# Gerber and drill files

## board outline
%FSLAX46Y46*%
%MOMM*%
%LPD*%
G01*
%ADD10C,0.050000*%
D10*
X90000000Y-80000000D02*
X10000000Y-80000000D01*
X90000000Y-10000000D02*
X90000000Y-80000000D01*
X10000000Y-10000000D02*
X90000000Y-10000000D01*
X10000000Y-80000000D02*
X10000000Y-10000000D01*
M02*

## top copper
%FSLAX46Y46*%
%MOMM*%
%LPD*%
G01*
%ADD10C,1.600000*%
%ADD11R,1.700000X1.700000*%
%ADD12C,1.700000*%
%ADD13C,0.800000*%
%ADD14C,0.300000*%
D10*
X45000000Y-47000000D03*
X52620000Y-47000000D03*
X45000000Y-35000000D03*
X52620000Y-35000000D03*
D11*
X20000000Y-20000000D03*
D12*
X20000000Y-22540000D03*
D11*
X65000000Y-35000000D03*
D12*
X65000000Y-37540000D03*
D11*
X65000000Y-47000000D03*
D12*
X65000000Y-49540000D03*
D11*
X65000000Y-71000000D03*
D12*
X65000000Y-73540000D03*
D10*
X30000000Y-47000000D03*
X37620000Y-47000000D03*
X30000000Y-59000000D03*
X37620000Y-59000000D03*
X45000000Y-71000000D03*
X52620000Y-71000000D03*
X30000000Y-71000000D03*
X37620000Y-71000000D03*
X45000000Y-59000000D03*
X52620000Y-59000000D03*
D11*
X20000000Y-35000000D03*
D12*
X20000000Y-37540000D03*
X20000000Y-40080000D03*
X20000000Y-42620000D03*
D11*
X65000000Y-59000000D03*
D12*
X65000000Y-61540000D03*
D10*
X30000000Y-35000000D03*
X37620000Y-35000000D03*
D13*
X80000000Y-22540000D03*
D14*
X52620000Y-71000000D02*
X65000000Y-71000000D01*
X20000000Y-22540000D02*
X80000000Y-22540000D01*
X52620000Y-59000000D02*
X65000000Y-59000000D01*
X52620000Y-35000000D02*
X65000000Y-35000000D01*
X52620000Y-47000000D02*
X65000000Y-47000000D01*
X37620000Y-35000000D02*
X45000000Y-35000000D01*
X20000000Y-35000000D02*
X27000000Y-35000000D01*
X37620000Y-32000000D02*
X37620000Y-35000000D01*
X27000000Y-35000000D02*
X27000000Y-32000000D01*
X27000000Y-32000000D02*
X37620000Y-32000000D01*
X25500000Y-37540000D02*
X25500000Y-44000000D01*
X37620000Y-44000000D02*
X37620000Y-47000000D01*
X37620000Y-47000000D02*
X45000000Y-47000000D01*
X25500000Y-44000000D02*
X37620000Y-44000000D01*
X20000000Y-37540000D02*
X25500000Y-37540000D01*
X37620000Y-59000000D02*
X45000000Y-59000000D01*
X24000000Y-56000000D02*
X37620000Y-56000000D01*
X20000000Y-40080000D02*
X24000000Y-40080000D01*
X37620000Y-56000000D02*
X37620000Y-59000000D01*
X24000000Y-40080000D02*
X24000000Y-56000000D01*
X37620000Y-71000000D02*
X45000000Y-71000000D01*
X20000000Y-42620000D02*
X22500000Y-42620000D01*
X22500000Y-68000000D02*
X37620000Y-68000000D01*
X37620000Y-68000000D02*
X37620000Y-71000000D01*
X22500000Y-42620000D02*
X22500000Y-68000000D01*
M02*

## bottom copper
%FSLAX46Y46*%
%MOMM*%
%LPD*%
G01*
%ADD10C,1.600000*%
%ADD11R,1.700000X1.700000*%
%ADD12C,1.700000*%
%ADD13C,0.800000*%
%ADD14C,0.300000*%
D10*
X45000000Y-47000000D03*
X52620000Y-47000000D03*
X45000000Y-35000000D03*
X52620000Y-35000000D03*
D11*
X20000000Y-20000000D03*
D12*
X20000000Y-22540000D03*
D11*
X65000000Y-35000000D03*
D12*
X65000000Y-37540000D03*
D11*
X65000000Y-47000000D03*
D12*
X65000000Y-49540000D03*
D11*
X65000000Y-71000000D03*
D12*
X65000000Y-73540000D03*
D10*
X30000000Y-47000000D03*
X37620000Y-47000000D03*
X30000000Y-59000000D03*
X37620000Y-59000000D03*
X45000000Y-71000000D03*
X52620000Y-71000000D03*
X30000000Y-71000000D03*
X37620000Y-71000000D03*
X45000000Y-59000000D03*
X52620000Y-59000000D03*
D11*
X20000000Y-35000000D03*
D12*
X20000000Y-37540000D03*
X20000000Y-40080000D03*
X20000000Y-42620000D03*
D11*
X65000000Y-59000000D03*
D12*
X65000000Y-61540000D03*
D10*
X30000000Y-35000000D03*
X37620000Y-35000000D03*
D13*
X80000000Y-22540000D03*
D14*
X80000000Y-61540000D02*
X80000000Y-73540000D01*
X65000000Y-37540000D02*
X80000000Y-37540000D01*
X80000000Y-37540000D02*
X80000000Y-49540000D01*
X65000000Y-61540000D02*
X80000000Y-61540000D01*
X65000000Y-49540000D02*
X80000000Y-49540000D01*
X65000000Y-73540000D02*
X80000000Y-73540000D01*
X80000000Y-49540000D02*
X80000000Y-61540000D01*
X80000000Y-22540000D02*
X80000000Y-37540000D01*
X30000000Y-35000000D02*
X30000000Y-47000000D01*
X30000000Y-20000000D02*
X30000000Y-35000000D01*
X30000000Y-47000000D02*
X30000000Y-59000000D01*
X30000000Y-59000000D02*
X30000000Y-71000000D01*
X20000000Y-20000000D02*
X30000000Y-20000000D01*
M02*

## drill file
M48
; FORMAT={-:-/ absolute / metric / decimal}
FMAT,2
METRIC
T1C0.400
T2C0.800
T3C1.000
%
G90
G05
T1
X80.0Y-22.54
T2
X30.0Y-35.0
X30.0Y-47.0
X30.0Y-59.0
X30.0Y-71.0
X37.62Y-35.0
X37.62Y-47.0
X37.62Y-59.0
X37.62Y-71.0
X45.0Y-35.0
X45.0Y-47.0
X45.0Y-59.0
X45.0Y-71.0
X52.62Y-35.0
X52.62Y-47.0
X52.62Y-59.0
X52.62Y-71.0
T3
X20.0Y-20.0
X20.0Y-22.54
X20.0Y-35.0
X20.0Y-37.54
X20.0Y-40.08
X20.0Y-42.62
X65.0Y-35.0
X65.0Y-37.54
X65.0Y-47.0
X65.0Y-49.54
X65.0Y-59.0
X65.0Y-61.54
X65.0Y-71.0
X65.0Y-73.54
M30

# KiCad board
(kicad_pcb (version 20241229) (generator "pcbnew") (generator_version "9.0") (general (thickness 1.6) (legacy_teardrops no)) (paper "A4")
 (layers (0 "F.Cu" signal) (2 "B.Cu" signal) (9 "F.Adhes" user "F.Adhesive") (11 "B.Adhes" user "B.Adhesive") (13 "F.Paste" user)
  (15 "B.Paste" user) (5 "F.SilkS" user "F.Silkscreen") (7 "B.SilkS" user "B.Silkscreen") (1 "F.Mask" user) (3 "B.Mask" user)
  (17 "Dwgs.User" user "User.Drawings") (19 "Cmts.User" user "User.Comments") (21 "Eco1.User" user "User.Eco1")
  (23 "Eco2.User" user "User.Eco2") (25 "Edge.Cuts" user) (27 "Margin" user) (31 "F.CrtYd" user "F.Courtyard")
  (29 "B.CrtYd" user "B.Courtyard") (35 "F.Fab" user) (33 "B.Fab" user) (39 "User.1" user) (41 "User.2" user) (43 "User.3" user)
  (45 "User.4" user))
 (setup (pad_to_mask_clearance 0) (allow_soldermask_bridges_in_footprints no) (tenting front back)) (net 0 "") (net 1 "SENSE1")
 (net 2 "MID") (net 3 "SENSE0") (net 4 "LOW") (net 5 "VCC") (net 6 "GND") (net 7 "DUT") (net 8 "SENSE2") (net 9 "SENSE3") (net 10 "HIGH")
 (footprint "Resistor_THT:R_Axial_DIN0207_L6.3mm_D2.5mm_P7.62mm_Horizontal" (layer "F.Cu") (at 45 47)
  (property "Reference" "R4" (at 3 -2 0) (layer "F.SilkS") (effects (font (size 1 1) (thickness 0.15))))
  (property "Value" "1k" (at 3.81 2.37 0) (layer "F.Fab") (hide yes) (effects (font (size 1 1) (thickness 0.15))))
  (pad "1" thru_hole circle (at 0 0) (size 1.6 1.6) (drill 0.8) (layers "*.Cu" "*.Mask") (remove_unused_layers no) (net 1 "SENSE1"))
  (pad "2" thru_hole circle (at 7.62 0) (size 1.6 1.6) (drill 0.8) (layers "*.Cu" "*.Mask") (remove_unused_layers no) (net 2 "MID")))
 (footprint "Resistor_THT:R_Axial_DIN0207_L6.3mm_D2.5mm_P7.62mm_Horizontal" (layer "F.Cu") (at 45 35)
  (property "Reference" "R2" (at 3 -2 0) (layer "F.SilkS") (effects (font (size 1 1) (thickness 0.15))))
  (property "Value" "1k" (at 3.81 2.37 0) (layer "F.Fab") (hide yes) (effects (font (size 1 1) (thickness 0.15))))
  (pad "1" thru_hole circle (at 0 0) (size 1.6 1.6) (drill 0.8) (layers "*.Cu" "*.Mask") (remove_unused_layers no) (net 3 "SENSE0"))
  (pad "2" thru_hole circle (at 7.62 0) (size 1.6 1.6) (drill 0.8) (layers "*.Cu" "*.Mask") (remove_unused_layers no) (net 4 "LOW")))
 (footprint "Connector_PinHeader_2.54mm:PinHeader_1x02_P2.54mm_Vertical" (layer "F.Cu") (at 20 20)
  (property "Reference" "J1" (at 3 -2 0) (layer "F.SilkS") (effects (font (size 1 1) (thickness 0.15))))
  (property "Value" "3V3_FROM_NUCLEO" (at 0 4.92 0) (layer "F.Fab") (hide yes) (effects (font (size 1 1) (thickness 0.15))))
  (pad "1" thru_hole rect (at 0 0) (size 1.7 1.7) (drill 1) (layers "*.Cu" "*.Mask") (remove_unused_layers no) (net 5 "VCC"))
  (pad "2" thru_hole circle (at 0 2.54) (size 1.7 1.7) (drill 1) (layers "*.Cu" "*.Mask") (remove_unused_layers no) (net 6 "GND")))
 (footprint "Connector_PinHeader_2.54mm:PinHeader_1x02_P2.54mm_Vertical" (layer "F.Cu") (at 65 35)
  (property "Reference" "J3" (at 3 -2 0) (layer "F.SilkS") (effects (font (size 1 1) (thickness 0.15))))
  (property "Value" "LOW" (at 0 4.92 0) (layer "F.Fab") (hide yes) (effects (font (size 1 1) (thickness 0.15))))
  (pad "1" thru_hole rect (at 0 0) (size 1.7 1.7) (drill 1) (layers "*.Cu" "*.Mask") (remove_unused_layers no) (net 4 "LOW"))
  (pad "2" thru_hole circle (at 0 2.54) (size 1.7 1.7) (drill 1) (layers "*.Cu" "*.Mask") (remove_unused_layers no) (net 6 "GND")))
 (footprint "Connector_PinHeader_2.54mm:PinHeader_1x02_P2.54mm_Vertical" (layer "F.Cu") (at 65 47)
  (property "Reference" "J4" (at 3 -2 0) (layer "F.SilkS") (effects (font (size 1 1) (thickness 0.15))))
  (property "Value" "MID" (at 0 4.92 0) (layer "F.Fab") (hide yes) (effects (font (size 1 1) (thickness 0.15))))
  (pad "1" thru_hole rect (at 0 0) (size 1.7 1.7) (drill 1) (layers "*.Cu" "*.Mask") (remove_unused_layers no) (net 2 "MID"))
  (pad "2" thru_hole circle (at 0 2.54) (size 1.7 1.7) (drill 1) (layers "*.Cu" "*.Mask") (remove_unused_layers no) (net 6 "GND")))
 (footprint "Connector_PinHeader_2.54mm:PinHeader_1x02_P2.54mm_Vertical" (layer "F.Cu") (at 65 71)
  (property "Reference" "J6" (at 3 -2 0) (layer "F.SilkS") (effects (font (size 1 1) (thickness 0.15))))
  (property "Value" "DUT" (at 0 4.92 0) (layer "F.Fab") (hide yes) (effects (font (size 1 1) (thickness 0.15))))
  (pad "1" thru_hole rect (at 0 0) (size 1.7 1.7) (drill 1) (layers "*.Cu" "*.Mask") (remove_unused_layers no) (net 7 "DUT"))
  (pad "2" thru_hole circle (at 0 2.54) (size 1.7 1.7) (drill 1) (layers "*.Cu" "*.Mask") (remove_unused_layers no) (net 6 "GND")))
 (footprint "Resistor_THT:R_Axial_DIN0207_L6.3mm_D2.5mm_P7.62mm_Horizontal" (layer "F.Cu") (at 30 47)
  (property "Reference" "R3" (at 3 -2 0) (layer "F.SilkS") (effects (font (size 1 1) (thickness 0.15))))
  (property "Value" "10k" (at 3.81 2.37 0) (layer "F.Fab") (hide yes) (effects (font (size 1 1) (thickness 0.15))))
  (pad "1" thru_hole circle (at 0 0) (size 1.6 1.6) (drill 0.8) (layers "*.Cu" "*.Mask") (remove_unused_layers no) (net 5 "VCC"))
  (pad "2" thru_hole circle (at 7.62 0) (size 1.6 1.6) (drill 0.8) (layers "*.Cu" "*.Mask") (remove_unused_layers no) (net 1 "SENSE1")))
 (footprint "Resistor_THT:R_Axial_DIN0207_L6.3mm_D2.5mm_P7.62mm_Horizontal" (layer "F.Cu") (at 30 59)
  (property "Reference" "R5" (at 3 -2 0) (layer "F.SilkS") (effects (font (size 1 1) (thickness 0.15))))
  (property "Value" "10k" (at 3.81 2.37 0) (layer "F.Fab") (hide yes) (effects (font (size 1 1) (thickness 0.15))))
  (pad "1" thru_hole circle (at 0 0) (size 1.6 1.6) (drill 0.8) (layers "*.Cu" "*.Mask") (remove_unused_layers no) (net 5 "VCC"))
  (pad "2" thru_hole circle (at 7.62 0) (size 1.6 1.6) (drill 0.8) (layers "*.Cu" "*.Mask") (remove_unused_layers no) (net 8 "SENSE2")))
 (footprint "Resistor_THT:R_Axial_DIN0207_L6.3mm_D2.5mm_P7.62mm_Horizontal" (layer "F.Cu") (at 45 71)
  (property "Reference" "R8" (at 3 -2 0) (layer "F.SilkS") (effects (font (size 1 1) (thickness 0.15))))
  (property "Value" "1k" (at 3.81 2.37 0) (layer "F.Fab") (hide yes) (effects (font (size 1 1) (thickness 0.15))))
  (pad "1" thru_hole circle (at 0 0) (size 1.6 1.6) (drill 0.8) (layers "*.Cu" "*.Mask") (remove_unused_layers no) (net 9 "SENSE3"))
  (pad "2" thru_hole circle (at 7.62 0) (size 1.6 1.6) (drill 0.8) (layers "*.Cu" "*.Mask") (remove_unused_layers no) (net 7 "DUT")))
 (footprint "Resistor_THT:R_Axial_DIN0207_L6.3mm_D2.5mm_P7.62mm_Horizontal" (layer "F.Cu") (at 30 71)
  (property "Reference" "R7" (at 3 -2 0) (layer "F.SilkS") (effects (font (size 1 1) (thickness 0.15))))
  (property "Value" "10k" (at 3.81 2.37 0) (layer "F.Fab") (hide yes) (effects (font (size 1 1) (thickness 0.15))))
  (pad "1" thru_hole circle (at 0 0) (size 1.6 1.6) (drill 0.8) (layers "*.Cu" "*.Mask") (remove_unused_layers no) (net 5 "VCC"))
  (pad "2" thru_hole circle (at 7.62 0) (size 1.6 1.6) (drill 0.8) (layers "*.Cu" "*.Mask") (remove_unused_layers no) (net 9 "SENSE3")))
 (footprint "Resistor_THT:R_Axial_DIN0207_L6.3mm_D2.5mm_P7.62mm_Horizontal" (layer "F.Cu") (at 45 59)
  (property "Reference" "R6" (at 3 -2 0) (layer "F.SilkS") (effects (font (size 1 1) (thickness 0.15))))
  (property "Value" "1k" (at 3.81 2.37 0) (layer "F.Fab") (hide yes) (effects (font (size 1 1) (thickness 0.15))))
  (pad "1" thru_hole circle (at 0 0) (size 1.6 1.6) (drill 0.8) (layers "*.Cu" "*.Mask") (remove_unused_layers no) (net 8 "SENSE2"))
  (pad "2" thru_hole circle (at 7.62 0) (size 1.6 1.6) (drill 0.8) (layers "*.Cu" "*.Mask") (remove_unused_layers no) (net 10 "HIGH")))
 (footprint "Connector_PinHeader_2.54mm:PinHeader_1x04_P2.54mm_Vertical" (layer "F.Cu") (at 20 35)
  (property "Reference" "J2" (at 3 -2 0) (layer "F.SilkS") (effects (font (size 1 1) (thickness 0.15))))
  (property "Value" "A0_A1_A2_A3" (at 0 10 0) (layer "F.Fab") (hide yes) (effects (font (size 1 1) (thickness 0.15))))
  (pad "1" thru_hole rect (at 0 0) (size 1.7 1.7) (drill 1) (layers "*.Cu" "*.Mask") (remove_unused_layers no) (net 3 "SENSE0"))
  (pad "2" thru_hole circle (at 0 2.54) (size 1.7 1.7) (drill 1) (layers "*.Cu" "*.Mask") (remove_unused_layers no) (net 1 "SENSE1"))
  (pad "3" thru_hole circle (at 0 5.08) (size 1.7 1.7) (drill 1) (layers "*.Cu" "*.Mask") (remove_unused_layers no) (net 8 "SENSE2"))
  (pad "4" thru_hole circle (at 0 7.62) (size 1.7 1.7) (drill 1) (layers "*.Cu" "*.Mask") (remove_unused_layers no) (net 9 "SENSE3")))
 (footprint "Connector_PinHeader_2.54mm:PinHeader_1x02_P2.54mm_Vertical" (layer "F.Cu") (at 65 59)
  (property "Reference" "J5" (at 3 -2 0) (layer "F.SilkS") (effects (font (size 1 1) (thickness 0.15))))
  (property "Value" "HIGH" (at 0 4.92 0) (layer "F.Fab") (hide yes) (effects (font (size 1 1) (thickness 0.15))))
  (pad "1" thru_hole rect (at 0 0) (size 1.7 1.7) (drill 1) (layers "*.Cu" "*.Mask") (remove_unused_layers no) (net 10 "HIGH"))
  (pad "2" thru_hole circle (at 0 2.54) (size 1.7 1.7) (drill 1) (layers "*.Cu" "*.Mask") (remove_unused_layers no) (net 6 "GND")))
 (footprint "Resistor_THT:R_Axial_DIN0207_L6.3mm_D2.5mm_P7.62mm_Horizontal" (layer "F.Cu") (at 30 35)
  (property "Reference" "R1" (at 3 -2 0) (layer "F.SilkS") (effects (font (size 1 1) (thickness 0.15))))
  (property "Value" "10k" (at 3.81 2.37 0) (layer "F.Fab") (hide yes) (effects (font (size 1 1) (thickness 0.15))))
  (pad "1" thru_hole circle (at 0 0) (size 1.6 1.6) (drill 0.8) (layers "*.Cu" "*.Mask") (remove_unused_layers no) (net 5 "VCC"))
  (pad "2" thru_hole circle (at 7.62 0) (size 1.6 1.6) (drill 0.8) (layers "*.Cu" "*.Mask") (remove_unused_layers no) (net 3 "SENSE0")))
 (gr_line (start 90 80) (end 10 80) (stroke (width 0.05) (type default)) (layer "Edge.Cuts"))
 (gr_line (start 90 10) (end 90 80) (stroke (width 0.05) (type default)) (layer "Edge.Cuts"))
 (gr_line (start 10 10) (end 90 10) (stroke (width 0.05) (type default)) (layer "Edge.Cuts"))
 (gr_line (start 10 80) (end 10 10) (stroke (width 0.05) (type default)) (layer "Edge.Cuts"))
 (segment (start 52.62 71) (end 65 71) (width 0.3) (layer "F.Cu") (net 7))
 (segment (start 20 22.54) (end 80 22.54) (width 0.3) (layer "F.Cu") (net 6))
 (via (at 80 22.54) (size 0.8) (drill 0.4) (layers "F.Cu" "B.Cu") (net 6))
 (segment (start 80 61.54) (end 80 73.54) (width 0.3) (layer "B.Cu") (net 6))
 (segment (start 65 37.54) (end 80 37.54) (width 0.3) (layer "B.Cu") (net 6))
 (segment (start 80 37.54) (end 80 49.54) (width 0.3) (layer "B.Cu") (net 6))
 (segment (start 65 61.54) (end 80 61.54) (width 0.3) (layer "B.Cu") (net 6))
 (segment (start 65 49.54) (end 80 49.54) (width 0.3) (layer "B.Cu") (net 6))
 (segment (start 65 73.54) (end 80 73.54) (width 0.3) (layer "B.Cu") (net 6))
 (segment (start 80 49.54) (end 80 61.54) (width 0.3) (layer "B.Cu") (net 6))
 (segment (start 80 22.54) (end 80 37.54) (width 0.3) (layer "B.Cu") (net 6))
 (segment (start 52.62 59) (end 65 59) (width 0.3) (layer "F.Cu") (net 10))
 (segment (start 52.62 35) (end 65 35) (width 0.3) (layer "F.Cu") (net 4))
 (segment (start 52.62 47) (end 65 47) (width 0.3) (layer "F.Cu") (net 2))
 (segment (start 37.62 35) (end 45 35) (width 0.3) (layer "F.Cu") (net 3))
 (segment (start 20 35) (end 27 35) (width 0.3) (layer "F.Cu") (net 3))
 (segment (start 37.62 32) (end 37.62 35) (width 0.3) (layer "F.Cu") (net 3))
 (segment (start 27 35) (end 27 32) (width 0.3) (layer "F.Cu") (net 3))
 (segment (start 27 32) (end 37.62 32) (width 0.3) (layer "F.Cu") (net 3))
 (segment (start 25.5 37.54) (end 25.5 44) (width 0.3) (layer "F.Cu") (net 1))
 (segment (start 37.62 44) (end 37.62 47) (width 0.3) (layer "F.Cu") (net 1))
 (segment (start 37.62 47) (end 45 47) (width 0.3) (layer "F.Cu") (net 1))
 (segment (start 25.5 44) (end 37.62 44) (width 0.3) (layer "F.Cu") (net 1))
 (segment (start 20 37.54) (end 25.5 37.54) (width 0.3) (layer "F.Cu") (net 1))
 (segment (start 37.62 59) (end 45 59) (width 0.3) (layer "F.Cu") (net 8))
 (segment (start 24 56) (end 37.62 56) (width 0.3) (layer "F.Cu") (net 8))
 (segment (start 20 40.08) (end 24 40.08) (width 0.3) (layer "F.Cu") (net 8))
 (segment (start 37.62 56) (end 37.62 59) (width 0.3) (layer "F.Cu") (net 8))
 (segment (start 24 40.08) (end 24 56) (width 0.3) (layer "F.Cu") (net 8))
 (segment (start 37.62 71) (end 45 71) (width 0.3) (layer "F.Cu") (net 9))
 (segment (start 20 42.62) (end 22.5 42.62) (width 0.3) (layer "F.Cu") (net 9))
 (segment (start 22.5 68) (end 37.62 68) (width 0.3) (layer "F.Cu") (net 9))
 (segment (start 37.62 68) (end 37.62 71) (width 0.3) (layer "F.Cu") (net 9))
 (segment (start 22.5 42.62) (end 22.5 68) (width 0.3) (layer "F.Cu") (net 9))
 (segment (start 30 35) (end 30 47) (width 0.3) (layer "B.Cu") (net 5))
 (segment (start 30 20) (end 30 35) (width 0.3) (layer "B.Cu") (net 5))
 (segment (start 30 47) (end 30 59) (width 0.3) (layer "B.Cu") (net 5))
 (segment (start 30 59) (end 30 71) (width 0.3) (layer "B.Cu") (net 5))
 (segment (start 20 20) (end 30 20) (width 0.3) (layer "B.Cu") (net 5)))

